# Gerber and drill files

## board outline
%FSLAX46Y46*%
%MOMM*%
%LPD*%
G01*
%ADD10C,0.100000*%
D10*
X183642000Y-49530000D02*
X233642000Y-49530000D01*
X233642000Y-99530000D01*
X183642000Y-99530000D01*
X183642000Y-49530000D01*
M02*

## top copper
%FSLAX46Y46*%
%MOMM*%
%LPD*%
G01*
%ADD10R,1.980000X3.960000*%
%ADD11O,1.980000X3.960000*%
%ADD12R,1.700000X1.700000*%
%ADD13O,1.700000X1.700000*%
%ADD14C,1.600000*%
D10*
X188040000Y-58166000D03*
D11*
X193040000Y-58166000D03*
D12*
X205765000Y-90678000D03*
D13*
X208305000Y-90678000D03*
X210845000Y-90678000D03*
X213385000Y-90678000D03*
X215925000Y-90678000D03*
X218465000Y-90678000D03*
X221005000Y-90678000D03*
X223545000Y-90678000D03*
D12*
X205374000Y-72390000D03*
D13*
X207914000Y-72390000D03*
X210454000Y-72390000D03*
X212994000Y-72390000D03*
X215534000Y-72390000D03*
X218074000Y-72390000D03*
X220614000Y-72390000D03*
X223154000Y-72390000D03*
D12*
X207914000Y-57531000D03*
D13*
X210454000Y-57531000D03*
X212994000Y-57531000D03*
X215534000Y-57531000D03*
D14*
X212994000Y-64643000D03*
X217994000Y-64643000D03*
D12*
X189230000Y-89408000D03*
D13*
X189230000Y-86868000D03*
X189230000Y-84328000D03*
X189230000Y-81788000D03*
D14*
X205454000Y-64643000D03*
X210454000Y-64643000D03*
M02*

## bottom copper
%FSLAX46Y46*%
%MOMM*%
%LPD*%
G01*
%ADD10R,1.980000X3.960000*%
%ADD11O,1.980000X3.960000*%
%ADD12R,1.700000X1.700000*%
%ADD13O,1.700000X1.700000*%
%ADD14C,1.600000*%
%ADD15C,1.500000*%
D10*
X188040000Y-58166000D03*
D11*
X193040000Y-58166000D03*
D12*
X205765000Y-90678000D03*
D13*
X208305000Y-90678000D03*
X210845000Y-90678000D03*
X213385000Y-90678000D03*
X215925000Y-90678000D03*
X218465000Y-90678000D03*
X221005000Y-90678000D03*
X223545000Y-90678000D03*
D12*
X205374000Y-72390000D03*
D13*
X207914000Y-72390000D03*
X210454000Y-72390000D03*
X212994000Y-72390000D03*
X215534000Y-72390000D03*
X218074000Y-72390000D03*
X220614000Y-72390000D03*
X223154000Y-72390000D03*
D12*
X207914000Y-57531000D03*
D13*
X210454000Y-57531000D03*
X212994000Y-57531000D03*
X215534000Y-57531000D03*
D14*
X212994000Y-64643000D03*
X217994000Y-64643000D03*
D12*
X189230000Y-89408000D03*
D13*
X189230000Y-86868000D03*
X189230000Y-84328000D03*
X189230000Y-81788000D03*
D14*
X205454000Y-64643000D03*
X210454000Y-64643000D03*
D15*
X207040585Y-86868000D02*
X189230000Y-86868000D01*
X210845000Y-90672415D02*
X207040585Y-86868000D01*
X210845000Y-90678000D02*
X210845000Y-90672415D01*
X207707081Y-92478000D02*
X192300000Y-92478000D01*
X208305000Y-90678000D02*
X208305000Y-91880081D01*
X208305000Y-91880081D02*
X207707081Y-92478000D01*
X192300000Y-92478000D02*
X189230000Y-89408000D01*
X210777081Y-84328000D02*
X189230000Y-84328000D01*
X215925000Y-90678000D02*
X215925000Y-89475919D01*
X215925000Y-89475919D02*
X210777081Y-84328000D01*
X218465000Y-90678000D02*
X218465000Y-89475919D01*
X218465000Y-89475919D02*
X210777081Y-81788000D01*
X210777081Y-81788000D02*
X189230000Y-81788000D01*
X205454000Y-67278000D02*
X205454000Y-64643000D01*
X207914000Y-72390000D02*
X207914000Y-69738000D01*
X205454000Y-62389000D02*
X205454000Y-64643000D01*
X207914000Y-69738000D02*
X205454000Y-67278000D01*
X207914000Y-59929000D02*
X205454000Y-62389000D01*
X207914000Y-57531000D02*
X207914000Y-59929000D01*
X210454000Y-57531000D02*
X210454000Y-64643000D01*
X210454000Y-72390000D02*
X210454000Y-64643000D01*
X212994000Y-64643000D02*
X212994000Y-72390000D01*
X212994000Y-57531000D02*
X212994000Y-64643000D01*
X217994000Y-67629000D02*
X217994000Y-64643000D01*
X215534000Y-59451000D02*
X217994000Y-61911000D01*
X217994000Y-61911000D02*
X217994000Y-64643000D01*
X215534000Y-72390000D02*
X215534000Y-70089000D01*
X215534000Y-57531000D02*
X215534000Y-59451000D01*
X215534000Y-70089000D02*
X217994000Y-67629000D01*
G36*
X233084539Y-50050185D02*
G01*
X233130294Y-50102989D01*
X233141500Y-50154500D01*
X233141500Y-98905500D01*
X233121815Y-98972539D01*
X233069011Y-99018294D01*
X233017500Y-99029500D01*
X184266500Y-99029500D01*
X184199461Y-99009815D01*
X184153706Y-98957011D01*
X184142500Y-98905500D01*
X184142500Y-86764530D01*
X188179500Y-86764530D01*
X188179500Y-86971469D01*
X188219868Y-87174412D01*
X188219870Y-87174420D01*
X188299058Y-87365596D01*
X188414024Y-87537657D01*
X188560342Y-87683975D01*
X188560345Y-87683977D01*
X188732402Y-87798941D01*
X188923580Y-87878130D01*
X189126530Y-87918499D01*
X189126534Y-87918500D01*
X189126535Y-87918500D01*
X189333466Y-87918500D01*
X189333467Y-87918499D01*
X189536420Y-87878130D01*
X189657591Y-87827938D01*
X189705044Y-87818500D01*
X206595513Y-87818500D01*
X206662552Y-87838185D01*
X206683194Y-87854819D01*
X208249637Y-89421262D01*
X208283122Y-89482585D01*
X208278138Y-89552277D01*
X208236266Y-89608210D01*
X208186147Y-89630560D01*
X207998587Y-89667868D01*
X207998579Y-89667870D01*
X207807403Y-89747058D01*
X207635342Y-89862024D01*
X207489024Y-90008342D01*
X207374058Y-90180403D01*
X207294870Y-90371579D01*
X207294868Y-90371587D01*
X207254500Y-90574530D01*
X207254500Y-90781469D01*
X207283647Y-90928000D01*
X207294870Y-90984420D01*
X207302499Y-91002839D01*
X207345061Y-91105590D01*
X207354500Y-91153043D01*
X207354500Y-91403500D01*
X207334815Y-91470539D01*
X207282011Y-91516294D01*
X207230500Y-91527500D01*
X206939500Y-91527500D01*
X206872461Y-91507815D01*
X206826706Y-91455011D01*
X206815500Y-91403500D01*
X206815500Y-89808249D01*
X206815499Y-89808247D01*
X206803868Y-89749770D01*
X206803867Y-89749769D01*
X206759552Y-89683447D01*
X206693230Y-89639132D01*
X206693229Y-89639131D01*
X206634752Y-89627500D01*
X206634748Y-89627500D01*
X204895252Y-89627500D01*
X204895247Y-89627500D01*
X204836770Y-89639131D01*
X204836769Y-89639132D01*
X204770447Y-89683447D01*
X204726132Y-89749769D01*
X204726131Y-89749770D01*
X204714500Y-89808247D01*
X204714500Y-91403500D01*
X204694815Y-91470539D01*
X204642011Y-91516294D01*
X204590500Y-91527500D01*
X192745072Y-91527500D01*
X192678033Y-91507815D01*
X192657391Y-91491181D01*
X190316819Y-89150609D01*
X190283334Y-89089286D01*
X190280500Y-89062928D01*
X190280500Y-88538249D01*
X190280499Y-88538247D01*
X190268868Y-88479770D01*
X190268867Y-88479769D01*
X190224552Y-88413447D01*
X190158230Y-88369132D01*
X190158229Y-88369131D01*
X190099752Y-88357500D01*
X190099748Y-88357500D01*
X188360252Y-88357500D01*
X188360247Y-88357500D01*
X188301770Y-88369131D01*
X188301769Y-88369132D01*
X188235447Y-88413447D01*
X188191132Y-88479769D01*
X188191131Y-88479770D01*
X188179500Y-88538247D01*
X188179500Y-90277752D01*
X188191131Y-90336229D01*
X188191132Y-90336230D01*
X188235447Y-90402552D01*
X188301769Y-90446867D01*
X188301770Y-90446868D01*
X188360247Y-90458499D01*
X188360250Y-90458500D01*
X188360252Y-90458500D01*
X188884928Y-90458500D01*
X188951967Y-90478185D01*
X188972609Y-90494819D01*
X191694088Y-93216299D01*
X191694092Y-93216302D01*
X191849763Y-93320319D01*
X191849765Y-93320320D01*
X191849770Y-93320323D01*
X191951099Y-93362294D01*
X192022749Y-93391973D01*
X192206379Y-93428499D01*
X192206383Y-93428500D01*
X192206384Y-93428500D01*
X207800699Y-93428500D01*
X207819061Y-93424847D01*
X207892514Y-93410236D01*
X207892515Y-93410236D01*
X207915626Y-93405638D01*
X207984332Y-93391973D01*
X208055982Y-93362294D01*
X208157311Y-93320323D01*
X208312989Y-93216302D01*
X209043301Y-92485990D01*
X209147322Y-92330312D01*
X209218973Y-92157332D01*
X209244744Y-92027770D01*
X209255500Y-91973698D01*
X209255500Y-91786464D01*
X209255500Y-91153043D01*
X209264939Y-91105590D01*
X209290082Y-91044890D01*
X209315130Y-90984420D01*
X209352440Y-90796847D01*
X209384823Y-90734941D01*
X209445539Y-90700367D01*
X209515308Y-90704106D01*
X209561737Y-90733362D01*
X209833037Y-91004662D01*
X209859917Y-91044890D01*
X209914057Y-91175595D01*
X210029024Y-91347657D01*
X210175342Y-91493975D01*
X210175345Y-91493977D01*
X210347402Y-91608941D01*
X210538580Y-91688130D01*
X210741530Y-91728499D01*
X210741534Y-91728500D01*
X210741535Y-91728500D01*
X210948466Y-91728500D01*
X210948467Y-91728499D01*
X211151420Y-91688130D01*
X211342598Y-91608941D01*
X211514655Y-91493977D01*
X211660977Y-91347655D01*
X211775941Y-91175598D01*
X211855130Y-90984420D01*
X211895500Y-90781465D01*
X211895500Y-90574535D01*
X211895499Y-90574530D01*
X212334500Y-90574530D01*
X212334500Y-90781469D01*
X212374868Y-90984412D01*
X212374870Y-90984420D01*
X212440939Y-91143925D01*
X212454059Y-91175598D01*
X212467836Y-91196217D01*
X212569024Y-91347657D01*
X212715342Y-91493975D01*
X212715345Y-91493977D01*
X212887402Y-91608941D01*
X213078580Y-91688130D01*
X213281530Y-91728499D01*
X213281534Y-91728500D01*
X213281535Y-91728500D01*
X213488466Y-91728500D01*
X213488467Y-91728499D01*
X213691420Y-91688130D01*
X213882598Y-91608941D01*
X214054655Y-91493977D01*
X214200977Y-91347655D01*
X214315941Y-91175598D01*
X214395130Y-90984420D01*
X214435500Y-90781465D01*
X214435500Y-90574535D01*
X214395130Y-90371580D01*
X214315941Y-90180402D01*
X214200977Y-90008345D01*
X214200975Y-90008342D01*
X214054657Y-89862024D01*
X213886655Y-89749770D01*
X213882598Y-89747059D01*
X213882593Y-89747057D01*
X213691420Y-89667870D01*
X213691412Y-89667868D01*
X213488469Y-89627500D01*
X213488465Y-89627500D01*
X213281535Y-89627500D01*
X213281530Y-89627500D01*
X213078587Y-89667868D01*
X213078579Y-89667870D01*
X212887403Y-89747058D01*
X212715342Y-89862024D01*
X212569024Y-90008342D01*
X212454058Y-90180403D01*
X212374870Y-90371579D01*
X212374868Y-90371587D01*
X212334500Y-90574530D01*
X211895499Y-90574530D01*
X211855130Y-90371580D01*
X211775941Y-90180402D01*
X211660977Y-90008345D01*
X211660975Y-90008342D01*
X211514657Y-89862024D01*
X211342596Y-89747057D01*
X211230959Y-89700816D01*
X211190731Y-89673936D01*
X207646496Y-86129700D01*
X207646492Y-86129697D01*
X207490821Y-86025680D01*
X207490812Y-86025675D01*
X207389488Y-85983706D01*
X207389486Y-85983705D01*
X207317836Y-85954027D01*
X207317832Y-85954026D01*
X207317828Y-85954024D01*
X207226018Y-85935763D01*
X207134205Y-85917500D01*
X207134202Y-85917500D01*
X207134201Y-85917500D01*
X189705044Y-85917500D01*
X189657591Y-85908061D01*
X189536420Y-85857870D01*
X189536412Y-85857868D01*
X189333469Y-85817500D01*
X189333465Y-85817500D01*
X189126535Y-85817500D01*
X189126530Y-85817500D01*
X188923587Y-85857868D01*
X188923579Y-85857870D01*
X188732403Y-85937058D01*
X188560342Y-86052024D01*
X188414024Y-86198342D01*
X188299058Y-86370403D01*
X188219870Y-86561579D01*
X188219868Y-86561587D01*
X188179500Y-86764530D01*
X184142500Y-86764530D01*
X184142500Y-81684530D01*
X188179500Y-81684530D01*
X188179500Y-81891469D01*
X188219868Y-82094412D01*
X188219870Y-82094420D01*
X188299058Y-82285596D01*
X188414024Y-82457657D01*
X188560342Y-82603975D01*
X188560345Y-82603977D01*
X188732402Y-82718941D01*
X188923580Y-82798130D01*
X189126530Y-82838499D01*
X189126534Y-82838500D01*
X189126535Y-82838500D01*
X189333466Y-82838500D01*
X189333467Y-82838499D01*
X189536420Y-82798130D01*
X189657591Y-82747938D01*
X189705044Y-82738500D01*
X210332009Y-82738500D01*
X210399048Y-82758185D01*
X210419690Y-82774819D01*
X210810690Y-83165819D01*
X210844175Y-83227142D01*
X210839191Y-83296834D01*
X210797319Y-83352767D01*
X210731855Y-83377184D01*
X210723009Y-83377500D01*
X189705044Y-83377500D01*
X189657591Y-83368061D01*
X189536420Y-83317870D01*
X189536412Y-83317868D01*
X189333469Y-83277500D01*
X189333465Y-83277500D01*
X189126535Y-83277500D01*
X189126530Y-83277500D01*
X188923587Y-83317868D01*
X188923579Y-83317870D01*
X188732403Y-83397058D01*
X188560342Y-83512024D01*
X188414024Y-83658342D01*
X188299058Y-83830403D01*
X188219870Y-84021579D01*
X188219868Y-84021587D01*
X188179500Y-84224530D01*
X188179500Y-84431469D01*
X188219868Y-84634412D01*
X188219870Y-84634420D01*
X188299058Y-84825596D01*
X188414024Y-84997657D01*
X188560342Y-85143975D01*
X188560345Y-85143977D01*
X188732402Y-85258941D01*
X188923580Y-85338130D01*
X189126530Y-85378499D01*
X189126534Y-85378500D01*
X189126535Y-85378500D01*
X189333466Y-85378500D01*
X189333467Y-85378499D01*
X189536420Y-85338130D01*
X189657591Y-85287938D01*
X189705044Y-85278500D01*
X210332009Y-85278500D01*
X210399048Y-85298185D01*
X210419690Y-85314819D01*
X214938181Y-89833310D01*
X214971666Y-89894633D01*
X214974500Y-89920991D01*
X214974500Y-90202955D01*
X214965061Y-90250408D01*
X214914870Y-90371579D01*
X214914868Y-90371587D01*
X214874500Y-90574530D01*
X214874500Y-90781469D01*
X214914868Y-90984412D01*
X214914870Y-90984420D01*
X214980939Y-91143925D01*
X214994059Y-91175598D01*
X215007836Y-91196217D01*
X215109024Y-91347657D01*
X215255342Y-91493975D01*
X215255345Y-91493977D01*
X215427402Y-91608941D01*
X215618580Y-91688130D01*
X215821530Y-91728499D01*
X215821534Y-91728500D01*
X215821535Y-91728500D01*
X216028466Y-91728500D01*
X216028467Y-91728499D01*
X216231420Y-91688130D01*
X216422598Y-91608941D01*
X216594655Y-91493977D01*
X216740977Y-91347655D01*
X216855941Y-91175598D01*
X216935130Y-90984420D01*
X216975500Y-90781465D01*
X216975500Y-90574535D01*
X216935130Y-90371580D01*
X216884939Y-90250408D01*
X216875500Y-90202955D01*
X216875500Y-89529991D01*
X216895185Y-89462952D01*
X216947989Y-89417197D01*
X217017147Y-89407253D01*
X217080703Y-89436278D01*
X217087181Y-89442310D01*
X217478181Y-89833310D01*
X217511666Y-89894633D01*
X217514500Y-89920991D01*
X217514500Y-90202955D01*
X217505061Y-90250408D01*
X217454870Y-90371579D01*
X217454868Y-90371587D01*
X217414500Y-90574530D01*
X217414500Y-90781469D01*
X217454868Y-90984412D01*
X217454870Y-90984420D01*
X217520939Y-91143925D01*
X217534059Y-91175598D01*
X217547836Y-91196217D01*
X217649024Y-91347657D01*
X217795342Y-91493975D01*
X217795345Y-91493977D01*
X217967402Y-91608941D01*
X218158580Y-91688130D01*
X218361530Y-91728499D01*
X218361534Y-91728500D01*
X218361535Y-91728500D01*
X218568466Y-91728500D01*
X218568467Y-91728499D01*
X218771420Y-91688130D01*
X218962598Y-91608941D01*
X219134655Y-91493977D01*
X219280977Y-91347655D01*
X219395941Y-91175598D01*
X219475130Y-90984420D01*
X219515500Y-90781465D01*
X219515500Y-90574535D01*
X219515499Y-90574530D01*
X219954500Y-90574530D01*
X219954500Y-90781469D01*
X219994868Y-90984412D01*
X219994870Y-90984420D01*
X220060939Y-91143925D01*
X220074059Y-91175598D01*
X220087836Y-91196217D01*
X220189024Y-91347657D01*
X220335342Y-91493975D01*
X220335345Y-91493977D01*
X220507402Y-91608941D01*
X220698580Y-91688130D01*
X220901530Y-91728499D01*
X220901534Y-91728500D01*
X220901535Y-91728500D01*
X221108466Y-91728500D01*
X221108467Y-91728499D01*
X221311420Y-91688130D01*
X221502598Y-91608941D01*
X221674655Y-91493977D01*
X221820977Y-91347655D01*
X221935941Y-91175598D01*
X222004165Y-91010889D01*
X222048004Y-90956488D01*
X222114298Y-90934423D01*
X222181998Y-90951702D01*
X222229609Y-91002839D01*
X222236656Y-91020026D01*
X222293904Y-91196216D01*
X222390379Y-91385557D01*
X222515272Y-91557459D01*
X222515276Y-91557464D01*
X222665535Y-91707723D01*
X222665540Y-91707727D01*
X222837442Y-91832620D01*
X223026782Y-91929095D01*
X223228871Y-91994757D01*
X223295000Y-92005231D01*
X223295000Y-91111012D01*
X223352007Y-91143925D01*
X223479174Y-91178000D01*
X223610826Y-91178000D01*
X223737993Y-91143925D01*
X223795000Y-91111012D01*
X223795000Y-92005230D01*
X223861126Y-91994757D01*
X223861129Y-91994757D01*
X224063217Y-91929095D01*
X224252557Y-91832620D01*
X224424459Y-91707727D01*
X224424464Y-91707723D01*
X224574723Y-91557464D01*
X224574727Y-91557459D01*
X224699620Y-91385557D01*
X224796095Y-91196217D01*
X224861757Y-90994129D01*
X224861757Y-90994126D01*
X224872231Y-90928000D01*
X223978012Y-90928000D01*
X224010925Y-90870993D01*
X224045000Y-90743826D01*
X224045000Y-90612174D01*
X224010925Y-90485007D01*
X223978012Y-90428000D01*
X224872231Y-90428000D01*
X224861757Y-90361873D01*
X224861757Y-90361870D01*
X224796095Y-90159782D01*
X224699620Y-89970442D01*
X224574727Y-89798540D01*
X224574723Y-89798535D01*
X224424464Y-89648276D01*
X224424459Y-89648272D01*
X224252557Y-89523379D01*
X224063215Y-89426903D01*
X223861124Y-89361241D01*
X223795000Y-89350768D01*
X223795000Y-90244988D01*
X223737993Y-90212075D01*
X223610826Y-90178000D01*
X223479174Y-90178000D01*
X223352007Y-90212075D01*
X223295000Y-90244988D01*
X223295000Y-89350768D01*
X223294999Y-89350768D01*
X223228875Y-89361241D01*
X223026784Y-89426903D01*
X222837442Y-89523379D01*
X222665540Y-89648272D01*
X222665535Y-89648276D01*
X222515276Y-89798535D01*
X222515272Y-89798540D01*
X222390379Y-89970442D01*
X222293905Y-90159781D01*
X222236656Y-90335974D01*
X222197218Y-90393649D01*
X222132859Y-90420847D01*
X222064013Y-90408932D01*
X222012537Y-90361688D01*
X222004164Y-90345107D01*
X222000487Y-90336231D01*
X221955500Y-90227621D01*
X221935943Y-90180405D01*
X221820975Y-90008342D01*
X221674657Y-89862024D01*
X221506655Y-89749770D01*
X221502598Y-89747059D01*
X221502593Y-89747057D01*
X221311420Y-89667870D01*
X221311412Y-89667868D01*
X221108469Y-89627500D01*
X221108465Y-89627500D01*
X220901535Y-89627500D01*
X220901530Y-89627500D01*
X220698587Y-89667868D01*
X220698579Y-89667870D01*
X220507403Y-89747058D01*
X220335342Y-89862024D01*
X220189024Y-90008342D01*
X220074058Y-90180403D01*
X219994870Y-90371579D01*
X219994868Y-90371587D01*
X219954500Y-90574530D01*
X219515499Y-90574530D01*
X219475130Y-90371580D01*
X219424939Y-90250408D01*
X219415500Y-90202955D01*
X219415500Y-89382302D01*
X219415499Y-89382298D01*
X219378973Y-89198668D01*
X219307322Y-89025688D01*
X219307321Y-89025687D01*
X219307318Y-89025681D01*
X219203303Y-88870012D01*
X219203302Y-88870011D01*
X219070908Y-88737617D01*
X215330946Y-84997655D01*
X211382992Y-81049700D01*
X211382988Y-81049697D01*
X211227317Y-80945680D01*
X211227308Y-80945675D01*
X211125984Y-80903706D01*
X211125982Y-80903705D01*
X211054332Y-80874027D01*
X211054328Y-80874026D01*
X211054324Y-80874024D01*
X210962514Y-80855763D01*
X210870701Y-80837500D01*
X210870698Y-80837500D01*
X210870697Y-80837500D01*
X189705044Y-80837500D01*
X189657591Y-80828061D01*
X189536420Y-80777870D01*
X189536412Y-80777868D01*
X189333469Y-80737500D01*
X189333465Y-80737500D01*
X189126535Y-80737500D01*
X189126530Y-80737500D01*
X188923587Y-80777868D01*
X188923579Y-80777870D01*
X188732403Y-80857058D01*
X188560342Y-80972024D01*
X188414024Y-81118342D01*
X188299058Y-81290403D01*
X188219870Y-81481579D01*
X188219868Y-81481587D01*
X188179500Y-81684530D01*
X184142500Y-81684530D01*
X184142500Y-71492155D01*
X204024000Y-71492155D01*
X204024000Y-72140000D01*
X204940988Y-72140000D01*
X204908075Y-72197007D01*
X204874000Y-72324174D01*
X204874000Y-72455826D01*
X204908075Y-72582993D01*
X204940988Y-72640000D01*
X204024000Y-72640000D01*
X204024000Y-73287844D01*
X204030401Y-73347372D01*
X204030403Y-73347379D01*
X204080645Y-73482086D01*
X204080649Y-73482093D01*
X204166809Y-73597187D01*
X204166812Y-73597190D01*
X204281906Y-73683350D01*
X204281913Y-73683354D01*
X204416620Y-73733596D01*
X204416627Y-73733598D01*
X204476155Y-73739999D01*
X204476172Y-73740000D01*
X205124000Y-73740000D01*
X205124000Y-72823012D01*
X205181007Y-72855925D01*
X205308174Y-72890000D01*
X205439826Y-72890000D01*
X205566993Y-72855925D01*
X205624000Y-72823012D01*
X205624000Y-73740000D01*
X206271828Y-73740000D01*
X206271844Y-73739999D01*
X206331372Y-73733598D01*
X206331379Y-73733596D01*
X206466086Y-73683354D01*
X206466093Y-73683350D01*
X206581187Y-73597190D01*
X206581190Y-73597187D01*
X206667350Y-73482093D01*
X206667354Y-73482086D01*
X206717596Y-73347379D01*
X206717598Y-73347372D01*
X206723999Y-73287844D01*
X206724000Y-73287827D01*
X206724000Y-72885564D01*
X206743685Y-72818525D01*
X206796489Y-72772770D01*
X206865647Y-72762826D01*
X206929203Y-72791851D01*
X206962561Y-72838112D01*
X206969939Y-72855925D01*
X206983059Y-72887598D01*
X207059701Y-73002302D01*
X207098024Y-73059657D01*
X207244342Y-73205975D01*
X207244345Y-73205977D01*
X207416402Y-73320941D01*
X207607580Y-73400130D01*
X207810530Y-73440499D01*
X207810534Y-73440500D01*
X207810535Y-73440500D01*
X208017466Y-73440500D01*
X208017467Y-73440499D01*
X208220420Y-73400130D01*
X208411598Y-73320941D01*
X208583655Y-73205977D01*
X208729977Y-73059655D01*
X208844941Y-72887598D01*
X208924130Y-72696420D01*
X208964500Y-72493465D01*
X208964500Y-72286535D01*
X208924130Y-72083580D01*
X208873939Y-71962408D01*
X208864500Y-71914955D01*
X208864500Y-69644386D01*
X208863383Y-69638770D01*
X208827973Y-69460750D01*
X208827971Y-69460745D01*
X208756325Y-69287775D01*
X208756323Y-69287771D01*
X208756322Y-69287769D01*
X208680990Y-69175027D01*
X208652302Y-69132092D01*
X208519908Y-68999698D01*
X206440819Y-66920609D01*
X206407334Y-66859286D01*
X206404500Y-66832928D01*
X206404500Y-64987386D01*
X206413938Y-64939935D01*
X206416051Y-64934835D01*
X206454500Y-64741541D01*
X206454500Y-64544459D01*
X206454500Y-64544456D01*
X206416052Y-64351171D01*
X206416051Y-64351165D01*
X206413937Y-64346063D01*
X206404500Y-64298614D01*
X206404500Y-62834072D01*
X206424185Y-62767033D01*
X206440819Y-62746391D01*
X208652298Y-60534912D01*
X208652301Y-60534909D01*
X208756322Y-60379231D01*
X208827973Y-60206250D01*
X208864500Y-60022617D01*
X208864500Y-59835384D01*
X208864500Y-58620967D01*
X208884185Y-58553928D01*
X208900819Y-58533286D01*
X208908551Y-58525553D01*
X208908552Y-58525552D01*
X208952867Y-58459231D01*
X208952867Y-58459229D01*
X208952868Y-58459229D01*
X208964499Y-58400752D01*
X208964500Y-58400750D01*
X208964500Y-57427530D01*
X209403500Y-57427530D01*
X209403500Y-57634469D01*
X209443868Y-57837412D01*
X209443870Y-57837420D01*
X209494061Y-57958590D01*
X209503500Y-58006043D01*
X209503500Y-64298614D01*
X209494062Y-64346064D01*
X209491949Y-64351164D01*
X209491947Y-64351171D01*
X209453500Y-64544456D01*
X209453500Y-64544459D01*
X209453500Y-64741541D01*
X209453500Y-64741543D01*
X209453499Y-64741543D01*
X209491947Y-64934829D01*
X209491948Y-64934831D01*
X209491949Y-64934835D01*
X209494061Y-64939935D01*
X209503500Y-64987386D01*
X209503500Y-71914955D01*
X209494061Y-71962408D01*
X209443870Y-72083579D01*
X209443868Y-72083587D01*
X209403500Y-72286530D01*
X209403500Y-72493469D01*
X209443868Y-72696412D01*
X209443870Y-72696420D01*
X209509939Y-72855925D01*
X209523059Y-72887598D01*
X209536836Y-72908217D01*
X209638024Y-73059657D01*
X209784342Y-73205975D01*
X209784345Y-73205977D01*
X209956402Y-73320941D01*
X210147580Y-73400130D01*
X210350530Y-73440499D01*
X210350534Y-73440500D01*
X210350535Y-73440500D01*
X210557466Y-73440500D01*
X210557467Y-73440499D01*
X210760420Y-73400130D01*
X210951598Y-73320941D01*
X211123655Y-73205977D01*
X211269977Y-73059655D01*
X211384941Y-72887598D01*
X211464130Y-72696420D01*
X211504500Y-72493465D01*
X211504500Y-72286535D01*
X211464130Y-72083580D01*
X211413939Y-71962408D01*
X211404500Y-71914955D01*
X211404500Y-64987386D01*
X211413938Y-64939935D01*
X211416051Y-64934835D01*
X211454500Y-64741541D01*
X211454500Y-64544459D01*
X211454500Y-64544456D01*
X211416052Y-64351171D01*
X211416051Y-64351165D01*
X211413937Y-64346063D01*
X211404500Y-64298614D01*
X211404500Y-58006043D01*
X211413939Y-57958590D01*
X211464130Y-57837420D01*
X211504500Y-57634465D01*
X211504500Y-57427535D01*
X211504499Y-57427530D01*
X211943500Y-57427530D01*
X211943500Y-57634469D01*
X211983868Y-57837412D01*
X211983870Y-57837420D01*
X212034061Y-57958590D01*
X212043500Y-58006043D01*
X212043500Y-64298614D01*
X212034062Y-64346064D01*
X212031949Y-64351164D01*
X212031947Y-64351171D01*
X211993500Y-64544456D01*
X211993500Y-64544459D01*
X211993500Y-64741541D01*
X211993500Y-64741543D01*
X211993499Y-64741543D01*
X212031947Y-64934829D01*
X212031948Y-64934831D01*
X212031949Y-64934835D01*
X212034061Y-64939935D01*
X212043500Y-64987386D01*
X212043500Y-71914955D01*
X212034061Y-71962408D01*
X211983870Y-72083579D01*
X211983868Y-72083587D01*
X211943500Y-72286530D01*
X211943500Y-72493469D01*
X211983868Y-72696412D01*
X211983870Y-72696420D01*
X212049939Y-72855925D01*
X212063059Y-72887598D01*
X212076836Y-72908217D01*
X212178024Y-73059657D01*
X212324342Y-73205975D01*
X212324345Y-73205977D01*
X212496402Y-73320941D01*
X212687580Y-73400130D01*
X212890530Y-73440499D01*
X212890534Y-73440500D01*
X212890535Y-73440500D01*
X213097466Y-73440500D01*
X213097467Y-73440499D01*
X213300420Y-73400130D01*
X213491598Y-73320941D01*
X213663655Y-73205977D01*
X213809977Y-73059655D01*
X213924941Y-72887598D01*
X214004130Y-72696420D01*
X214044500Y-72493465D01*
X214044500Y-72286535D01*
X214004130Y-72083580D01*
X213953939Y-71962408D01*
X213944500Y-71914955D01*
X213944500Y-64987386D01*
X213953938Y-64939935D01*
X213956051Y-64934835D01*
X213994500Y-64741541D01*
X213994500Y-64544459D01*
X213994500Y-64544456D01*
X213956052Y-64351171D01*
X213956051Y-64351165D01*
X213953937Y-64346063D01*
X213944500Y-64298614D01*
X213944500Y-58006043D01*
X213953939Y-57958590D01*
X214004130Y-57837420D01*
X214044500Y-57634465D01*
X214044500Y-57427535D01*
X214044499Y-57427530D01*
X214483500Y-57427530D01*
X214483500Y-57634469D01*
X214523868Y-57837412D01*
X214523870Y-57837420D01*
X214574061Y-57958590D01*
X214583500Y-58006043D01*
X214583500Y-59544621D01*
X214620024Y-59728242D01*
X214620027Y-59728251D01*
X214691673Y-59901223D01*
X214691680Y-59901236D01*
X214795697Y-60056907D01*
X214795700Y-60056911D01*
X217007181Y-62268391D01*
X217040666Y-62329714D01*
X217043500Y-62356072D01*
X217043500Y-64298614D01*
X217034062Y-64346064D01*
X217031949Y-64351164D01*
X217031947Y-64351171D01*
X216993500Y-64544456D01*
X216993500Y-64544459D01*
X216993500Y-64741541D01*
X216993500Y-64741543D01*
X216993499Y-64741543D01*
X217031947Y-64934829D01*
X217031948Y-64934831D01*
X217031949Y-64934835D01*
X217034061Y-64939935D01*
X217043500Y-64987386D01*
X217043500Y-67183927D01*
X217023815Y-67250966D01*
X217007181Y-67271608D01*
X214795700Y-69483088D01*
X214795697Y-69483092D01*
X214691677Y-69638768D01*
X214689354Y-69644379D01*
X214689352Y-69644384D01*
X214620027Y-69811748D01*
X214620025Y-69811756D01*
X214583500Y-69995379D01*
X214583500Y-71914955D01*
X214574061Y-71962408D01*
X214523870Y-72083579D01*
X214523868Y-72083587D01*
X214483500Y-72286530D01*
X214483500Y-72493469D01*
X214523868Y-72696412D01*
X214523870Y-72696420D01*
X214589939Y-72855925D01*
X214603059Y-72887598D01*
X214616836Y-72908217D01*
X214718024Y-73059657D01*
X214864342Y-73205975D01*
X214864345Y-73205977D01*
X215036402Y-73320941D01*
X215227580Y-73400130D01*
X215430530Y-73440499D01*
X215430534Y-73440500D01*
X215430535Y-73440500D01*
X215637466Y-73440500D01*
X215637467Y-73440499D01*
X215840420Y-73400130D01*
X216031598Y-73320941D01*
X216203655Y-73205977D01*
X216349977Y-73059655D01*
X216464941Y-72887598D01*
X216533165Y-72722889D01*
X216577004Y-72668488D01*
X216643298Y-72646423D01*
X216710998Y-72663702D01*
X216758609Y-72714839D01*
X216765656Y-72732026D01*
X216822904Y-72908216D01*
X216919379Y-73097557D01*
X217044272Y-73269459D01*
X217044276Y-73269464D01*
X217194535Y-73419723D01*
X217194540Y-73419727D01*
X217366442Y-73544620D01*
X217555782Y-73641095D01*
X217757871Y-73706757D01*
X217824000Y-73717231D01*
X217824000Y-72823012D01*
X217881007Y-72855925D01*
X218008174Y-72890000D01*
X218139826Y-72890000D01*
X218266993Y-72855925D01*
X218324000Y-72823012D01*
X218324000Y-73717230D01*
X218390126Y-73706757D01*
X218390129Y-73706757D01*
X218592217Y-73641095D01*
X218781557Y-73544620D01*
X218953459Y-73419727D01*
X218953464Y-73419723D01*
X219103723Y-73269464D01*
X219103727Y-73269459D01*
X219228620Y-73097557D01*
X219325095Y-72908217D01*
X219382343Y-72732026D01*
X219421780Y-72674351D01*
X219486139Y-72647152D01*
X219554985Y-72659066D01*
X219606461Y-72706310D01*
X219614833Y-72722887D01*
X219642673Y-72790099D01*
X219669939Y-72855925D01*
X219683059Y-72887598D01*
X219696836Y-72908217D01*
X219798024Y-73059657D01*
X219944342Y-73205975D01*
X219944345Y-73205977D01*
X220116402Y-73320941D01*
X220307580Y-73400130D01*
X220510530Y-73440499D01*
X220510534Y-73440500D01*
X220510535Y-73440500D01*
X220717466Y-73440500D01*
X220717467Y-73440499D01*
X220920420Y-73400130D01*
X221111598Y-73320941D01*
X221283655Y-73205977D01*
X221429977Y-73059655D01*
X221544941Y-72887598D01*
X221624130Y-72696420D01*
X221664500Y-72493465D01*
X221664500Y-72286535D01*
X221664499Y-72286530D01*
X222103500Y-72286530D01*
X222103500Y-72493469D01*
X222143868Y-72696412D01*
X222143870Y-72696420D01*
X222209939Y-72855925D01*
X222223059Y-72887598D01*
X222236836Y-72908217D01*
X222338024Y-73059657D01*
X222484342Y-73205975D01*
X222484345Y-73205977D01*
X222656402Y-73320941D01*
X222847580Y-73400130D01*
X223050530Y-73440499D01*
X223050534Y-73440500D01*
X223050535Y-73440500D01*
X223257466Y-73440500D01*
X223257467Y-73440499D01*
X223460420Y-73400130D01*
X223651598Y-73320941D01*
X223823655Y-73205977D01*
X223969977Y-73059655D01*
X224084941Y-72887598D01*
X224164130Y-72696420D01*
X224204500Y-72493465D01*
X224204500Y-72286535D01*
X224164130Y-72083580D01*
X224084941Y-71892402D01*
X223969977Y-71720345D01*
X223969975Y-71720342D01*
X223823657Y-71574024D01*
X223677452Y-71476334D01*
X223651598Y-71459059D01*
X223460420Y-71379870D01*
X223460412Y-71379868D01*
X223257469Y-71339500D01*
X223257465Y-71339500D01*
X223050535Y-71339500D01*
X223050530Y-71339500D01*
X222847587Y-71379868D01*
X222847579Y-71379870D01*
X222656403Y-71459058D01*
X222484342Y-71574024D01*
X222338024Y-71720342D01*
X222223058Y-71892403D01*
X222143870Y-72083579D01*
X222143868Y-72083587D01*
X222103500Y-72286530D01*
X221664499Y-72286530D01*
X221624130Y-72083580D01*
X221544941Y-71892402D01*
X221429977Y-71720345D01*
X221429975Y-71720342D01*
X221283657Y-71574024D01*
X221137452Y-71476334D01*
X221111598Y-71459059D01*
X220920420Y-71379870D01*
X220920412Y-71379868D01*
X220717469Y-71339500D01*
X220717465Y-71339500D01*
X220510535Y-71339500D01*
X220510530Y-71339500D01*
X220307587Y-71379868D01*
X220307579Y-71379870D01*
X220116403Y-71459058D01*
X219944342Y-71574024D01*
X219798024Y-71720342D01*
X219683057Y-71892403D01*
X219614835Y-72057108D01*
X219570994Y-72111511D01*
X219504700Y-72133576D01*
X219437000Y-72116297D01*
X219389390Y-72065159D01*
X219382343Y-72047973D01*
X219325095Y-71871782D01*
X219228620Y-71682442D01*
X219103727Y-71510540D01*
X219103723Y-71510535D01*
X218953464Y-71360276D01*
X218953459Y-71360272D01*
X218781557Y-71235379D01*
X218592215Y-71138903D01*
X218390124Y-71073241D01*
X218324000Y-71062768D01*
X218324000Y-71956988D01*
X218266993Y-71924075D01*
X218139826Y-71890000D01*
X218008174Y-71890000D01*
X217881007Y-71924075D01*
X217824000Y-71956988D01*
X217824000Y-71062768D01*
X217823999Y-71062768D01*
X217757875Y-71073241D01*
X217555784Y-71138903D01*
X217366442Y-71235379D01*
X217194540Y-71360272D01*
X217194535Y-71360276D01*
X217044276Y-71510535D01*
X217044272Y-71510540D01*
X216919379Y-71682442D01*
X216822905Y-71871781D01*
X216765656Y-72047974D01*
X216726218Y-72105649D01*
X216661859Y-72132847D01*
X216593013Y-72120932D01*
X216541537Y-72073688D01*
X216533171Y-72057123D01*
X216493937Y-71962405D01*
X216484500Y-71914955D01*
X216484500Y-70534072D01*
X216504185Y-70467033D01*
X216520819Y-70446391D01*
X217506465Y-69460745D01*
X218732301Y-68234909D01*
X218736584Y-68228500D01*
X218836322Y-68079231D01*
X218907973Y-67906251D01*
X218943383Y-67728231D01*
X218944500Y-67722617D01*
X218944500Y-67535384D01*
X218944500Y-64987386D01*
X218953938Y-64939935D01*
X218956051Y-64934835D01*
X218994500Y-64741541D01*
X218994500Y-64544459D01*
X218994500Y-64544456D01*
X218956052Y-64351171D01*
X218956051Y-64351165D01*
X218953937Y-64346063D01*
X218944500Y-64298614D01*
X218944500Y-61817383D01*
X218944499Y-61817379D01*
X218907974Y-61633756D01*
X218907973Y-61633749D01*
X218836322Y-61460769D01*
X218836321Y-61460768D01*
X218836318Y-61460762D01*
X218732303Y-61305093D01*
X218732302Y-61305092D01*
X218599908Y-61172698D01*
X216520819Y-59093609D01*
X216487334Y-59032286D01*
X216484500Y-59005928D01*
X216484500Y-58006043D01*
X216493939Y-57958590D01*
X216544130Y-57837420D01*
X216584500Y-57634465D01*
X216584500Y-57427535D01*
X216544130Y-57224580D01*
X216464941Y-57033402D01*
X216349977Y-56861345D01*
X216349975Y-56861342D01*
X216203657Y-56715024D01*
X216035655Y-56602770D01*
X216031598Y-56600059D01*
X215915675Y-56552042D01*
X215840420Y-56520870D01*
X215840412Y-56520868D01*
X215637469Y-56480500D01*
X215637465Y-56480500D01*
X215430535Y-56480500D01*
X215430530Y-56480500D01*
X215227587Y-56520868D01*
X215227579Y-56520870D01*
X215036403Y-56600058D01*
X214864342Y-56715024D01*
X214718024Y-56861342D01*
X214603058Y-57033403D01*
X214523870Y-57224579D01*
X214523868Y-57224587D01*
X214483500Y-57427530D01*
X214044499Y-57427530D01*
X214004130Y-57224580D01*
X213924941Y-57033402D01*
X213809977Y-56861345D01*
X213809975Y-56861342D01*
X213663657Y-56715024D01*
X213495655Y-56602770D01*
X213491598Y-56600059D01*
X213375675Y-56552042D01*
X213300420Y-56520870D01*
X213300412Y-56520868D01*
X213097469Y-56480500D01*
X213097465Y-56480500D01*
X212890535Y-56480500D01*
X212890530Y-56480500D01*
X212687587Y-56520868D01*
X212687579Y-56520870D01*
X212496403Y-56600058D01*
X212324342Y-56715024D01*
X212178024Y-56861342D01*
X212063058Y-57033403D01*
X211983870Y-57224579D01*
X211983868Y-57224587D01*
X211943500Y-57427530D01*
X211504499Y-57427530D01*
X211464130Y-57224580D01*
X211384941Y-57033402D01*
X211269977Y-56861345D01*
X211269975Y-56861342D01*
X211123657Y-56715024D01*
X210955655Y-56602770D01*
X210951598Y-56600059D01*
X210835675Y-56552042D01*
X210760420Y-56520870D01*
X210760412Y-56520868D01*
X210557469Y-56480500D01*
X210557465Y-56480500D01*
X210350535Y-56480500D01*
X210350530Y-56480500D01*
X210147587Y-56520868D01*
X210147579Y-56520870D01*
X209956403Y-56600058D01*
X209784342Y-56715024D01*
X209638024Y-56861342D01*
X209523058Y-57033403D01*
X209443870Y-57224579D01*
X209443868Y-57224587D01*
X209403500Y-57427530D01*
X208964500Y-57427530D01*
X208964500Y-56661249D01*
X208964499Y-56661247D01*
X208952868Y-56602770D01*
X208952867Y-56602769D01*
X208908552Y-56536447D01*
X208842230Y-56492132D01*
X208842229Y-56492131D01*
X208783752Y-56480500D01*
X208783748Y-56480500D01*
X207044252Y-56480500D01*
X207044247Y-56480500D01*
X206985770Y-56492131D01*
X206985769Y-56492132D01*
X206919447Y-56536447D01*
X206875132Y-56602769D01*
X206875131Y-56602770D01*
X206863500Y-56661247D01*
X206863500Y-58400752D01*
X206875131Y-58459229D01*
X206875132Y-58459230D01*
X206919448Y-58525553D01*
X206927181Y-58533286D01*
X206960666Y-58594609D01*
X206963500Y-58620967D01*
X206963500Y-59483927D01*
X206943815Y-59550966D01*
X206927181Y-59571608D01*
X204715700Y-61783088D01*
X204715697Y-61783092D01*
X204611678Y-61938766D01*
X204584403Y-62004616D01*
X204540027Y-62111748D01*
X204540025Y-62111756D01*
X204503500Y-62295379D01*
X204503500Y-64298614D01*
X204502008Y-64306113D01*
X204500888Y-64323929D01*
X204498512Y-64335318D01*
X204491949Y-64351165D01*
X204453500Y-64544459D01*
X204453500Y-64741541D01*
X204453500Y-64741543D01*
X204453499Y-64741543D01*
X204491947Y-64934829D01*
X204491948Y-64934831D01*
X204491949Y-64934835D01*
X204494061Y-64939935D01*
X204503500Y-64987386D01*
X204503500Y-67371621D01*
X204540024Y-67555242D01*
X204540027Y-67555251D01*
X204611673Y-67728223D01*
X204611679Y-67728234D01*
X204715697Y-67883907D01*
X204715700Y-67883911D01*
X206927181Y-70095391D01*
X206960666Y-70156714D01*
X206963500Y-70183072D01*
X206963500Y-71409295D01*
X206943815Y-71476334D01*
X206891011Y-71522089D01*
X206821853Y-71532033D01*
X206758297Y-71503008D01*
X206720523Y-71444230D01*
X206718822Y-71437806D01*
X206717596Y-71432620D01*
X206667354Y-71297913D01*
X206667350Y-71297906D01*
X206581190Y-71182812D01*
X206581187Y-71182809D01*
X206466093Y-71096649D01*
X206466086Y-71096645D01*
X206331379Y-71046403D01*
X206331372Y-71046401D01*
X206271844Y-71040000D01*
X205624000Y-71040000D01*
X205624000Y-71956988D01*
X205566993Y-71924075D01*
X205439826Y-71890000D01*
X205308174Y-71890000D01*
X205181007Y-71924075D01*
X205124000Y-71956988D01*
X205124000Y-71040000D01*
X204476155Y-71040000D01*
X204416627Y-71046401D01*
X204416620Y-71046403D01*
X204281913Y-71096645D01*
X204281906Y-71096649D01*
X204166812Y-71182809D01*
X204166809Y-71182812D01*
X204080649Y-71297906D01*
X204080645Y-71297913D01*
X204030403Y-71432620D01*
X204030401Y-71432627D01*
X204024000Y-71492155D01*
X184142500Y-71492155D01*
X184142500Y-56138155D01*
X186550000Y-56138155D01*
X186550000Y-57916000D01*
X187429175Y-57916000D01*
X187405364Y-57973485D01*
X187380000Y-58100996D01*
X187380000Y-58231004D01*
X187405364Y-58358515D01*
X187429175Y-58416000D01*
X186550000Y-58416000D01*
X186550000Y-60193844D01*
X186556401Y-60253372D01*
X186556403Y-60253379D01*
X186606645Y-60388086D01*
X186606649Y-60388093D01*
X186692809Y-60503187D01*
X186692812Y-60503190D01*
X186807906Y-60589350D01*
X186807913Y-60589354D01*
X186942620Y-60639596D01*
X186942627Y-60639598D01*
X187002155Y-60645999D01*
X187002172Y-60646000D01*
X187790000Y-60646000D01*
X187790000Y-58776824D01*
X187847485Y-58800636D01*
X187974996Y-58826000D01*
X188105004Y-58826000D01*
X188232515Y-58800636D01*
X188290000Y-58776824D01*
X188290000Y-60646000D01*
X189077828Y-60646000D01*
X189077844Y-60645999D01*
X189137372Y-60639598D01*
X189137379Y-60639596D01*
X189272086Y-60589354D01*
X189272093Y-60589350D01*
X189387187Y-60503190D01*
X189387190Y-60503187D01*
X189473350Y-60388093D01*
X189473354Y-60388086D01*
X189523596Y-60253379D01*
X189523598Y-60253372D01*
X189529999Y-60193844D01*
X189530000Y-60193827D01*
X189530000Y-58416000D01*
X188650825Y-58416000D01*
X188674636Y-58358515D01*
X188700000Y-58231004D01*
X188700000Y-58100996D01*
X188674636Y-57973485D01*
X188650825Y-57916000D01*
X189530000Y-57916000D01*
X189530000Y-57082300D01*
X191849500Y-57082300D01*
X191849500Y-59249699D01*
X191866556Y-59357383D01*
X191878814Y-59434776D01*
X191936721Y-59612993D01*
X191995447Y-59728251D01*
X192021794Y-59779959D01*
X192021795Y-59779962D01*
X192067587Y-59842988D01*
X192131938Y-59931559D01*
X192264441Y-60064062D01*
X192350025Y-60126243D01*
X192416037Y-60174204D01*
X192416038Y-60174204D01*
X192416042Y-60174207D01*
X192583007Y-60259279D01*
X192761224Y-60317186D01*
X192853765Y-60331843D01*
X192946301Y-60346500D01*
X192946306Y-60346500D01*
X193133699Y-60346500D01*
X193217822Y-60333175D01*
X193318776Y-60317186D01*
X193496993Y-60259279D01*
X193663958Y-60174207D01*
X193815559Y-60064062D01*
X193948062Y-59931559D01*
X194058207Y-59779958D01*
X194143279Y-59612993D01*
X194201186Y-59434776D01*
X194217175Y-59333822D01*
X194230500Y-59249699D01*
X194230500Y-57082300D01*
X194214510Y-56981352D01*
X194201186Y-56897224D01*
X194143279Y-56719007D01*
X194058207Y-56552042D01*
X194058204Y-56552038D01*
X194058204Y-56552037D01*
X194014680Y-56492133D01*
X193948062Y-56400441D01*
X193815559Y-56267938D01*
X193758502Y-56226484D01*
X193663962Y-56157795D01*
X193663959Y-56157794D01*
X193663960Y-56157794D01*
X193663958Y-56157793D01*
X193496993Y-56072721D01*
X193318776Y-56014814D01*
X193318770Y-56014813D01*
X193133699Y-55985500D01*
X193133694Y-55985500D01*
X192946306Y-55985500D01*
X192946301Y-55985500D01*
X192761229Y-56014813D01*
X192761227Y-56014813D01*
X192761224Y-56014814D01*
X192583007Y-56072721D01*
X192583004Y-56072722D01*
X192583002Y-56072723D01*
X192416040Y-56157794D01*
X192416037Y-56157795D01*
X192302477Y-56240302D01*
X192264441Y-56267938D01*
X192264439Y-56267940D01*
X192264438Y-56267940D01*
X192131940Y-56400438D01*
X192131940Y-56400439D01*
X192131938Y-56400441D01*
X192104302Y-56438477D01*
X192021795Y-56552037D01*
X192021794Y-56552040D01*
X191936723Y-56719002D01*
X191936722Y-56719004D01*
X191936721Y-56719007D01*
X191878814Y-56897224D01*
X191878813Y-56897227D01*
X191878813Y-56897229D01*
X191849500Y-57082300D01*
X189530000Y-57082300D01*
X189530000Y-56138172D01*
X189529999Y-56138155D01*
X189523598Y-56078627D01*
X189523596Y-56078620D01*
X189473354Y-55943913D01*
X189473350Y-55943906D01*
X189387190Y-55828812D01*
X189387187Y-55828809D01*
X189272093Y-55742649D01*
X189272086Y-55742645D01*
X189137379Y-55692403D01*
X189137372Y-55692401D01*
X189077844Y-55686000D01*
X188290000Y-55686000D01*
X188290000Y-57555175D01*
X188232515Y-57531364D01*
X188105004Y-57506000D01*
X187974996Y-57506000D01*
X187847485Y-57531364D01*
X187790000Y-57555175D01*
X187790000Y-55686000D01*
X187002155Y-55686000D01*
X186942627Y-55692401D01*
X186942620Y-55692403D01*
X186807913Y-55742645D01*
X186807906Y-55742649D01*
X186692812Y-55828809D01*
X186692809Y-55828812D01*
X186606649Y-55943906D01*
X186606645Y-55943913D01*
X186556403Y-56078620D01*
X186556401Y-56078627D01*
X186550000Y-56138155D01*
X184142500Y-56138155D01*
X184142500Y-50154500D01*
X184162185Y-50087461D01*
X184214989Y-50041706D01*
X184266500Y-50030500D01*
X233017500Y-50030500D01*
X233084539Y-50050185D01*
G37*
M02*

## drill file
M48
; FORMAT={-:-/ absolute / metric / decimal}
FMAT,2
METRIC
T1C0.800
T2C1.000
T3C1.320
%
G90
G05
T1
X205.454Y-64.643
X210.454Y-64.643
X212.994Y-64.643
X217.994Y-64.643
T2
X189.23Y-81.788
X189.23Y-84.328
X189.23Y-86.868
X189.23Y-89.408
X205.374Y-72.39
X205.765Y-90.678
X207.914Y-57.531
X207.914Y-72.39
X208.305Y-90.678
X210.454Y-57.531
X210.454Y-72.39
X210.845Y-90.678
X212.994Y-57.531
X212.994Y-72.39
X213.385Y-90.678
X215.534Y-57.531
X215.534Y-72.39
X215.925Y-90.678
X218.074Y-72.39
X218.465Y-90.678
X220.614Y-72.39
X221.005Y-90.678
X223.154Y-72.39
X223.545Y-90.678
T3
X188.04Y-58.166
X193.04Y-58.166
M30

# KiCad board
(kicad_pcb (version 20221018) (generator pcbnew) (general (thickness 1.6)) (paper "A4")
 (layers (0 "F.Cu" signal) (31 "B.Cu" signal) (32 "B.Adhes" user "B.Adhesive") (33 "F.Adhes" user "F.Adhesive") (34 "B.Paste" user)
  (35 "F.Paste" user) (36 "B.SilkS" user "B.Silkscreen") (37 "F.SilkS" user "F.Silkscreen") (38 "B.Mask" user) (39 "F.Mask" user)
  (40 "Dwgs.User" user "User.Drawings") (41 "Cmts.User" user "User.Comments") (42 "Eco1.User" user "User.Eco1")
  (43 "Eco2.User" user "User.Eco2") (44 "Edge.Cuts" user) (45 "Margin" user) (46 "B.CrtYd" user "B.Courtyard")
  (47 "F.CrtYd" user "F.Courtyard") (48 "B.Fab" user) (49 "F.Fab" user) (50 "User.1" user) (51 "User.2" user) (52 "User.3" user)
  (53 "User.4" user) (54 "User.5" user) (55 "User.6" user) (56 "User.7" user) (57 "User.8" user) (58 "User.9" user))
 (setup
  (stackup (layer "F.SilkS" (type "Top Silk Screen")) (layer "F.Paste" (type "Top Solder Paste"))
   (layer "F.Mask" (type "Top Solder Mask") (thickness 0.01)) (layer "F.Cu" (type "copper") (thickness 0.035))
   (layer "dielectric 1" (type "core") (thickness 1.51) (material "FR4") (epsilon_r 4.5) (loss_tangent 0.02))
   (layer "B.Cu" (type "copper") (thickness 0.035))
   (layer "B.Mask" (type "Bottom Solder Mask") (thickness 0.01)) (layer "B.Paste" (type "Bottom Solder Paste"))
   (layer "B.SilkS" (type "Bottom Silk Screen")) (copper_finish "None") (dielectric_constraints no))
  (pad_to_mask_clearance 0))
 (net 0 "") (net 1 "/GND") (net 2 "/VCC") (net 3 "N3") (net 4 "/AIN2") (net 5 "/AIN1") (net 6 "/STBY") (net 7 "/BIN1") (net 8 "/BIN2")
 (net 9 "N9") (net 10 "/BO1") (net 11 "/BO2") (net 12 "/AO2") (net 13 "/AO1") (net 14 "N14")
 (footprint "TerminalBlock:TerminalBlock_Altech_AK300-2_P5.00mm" (layer "F.Cu") (at 188.04 58.166)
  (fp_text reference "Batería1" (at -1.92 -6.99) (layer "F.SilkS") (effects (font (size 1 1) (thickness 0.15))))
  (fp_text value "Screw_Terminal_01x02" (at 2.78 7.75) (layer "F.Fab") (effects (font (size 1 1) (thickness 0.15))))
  (pad "1" thru_hole rect (at 0 0) (size 1.98 3.96) (drill 1.32) (layers "*.Cu" "*.Mask") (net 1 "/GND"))
  (pad "2" thru_hole oval (at 5 0) (size 1.98 3.96) (drill 1.32) (layers "*.Cu" "*.Mask") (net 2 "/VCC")))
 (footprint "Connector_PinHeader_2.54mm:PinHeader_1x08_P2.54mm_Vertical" (layer "F.Cu") (at 205.765 90.678 90)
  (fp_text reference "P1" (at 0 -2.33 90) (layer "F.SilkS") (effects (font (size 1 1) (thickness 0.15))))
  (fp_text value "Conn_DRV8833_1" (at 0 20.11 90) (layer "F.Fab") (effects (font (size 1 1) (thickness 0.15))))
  (pad "1" thru_hole rect (at 0 0 90) (size 1.7 1.7) (drill 1) (layers "*.Cu" "*.Mask") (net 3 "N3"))
  (pad "2" thru_hole oval (at 0 2.54 90) (size 1.7 1.7) (drill 1) (layers "*.Cu" "*.Mask") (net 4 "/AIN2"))
  (pad "3" thru_hole oval (at 0 5.08 90) (size 1.7 1.7) (drill 1) (layers "*.Cu" "*.Mask") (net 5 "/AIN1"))
  (pad "4" thru_hole oval (at 0 7.62 90) (size 1.7 1.7) (drill 1) (layers "*.Cu" "*.Mask") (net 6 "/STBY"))
  (pad "5" thru_hole oval (at 0 10.16 90) (size 1.7 1.7) (drill 1) (layers "*.Cu" "*.Mask") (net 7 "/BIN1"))
  (pad "6" thru_hole oval (at 0 12.7 90) (size 1.7 1.7) (drill 1) (layers "*.Cu" "*.Mask") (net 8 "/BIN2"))
  (pad "7" thru_hole oval (at 0 15.24 90) (size 1.7 1.7) (drill 1) (layers "*.Cu" "*.Mask") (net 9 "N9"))
  (pad "8" thru_hole oval (at 0 17.78 90) (size 1.7 1.7) (drill 1) (layers "*.Cu" "*.Mask") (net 1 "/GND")))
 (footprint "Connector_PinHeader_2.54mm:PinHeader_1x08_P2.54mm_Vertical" (layer "F.Cu") (at 205.374 72.39 90)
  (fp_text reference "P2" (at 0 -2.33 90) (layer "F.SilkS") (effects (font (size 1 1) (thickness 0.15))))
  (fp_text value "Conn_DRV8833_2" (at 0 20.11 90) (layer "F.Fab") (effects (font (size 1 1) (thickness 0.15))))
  (pad "1" thru_hole rect (at 0 0 90) (size 1.7 1.7) (drill 1) (layers "*.Cu" "*.Mask") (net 1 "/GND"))
  (pad "2" thru_hole oval (at 0 2.54 90) (size 1.7 1.7) (drill 1) (layers "*.Cu" "*.Mask") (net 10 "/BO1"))
  (pad "3" thru_hole oval (at 0 5.08 90) (size 1.7 1.7) (drill 1) (layers "*.Cu" "*.Mask") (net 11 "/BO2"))
  (pad "4" thru_hole oval (at 0 7.62 90) (size 1.7 1.7) (drill 1) (layers "*.Cu" "*.Mask") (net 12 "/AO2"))
  (pad "5" thru_hole oval (at 0 10.16 90) (size 1.7 1.7) (drill 1) (layers "*.Cu" "*.Mask") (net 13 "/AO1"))
  (pad "6" thru_hole oval (at 0 12.7 90) (size 1.7 1.7) (drill 1) (layers "*.Cu" "*.Mask") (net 1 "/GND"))
  (pad "7" thru_hole oval (at 0 15.24 90) (size 1.7 1.7) (drill 1) (layers "*.Cu" "*.Mask") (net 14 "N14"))
  (pad "8" thru_hole oval (at 0 17.78 90) (size 1.7 1.7) (drill 1) (layers "*.Cu" "*.Mask") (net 2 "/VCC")))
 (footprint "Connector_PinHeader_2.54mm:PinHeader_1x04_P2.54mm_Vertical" (layer "F.Cu") (at 207.914 57.531 90)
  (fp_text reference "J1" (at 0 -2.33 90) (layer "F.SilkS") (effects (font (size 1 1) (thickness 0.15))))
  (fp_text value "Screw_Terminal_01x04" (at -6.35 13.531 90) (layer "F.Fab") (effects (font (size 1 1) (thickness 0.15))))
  (pad "1" thru_hole rect (at 0 0 90) (size 1.7 1.7) (drill 1) (layers "*.Cu" "*.Mask") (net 10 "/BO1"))
  (pad "2" thru_hole oval (at 0 2.54 90) (size 1.7 1.7) (drill 1) (layers "*.Cu" "*.Mask") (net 11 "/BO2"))
  (pad "3" thru_hole oval (at 0 5.08 90) (size 1.7 1.7) (drill 1) (layers "*.Cu" "*.Mask") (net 12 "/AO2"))
  (pad "4" thru_hole oval (at 0 7.62 90) (size 1.7 1.7) (drill 1) (layers "*.Cu" "*.Mask") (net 13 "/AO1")))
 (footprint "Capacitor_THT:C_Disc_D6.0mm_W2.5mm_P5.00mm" (layer "F.Cu") (at 212.994 64.643)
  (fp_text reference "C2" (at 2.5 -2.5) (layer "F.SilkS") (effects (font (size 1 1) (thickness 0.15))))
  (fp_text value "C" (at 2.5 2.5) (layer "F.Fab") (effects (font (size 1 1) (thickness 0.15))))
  (pad "1" thru_hole circle (at 0 0) (size 1.6 1.6) (drill 0.8) (layers "*.Cu" "*.Mask") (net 12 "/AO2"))
  (pad "2" thru_hole circle (at 5 0) (size 1.6 1.6) (drill 0.8) (layers "*.Cu" "*.Mask") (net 13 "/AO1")))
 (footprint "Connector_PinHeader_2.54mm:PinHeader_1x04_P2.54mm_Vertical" (layer "F.Cu") (at 189.23 89.408 180)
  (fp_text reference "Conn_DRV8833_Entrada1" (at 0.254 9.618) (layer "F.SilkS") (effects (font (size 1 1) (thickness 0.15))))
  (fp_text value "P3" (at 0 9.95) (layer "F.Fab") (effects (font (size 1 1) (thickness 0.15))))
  (pad "1" thru_hole rect (at 0 0 180) (size 1.7 1.7) (drill 1) (layers "*.Cu" "*.Mask") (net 4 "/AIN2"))
  (pad "2" thru_hole oval (at 0 2.54 180) (size 1.7 1.7) (drill 1) (layers "*.Cu" "*.Mask") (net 5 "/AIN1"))
  (pad "3" thru_hole oval (at 0 5.08 180) (size 1.7 1.7) (drill 1) (layers "*.Cu" "*.Mask") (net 7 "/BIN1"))
  (pad "4" thru_hole oval (at 0 7.62 180) (size 1.7 1.7) (drill 1) (layers "*.Cu" "*.Mask") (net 8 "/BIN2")))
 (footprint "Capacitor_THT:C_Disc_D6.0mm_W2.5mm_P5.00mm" (layer "F.Cu") (at 205.454 64.643)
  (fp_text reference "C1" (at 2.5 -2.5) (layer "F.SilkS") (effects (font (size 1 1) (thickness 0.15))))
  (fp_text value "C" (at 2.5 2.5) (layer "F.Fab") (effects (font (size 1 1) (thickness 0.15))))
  (pad "1" thru_hole circle (at 0 0) (size 1.6 1.6) (drill 0.8) (layers "*.Cu" "*.Mask") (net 10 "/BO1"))
  (pad "2" thru_hole circle (at 5 0) (size 1.6 1.6) (drill 0.8) (layers "*.Cu" "*.Mask") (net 11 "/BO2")))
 (gr_rect (start 183.642 49.53) (end 233.642 99.53) (stroke (width 0.1) (type default)) (fill none) (layer "Edge.Cuts"))
 (segment (start 207.040585 86.868) (end 189.23 86.868) (width 1.5) (layer "B.Cu") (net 5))
 (segment (start 210.845 90.672415) (end 207.040585 86.868) (width 1.5) (layer "B.Cu") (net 5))
 (segment (start 210.845 90.678) (end 210.845 90.672415) (width 1.5) (layer "B.Cu") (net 5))
 (segment (start 207.707081 92.478) (end 192.3 92.478) (width 1.5) (layer "B.Cu") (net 4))
 (segment (start 208.305 90.678) (end 208.305 91.880081) (width 1.5) (layer "B.Cu") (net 4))
 (segment (start 208.305 91.880081) (end 207.707081 92.478) (width 1.5) (layer "B.Cu") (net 4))
 (segment (start 192.3 92.478) (end 189.23 89.408) (width 1.5) (layer "B.Cu") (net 4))
 (segment (start 210.777081 84.328) (end 189.23 84.328) (width 1.5) (layer "B.Cu") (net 7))
 (segment (start 215.925 90.678) (end 215.925 89.475919) (width 1.5) (layer "B.Cu") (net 7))
 (segment (start 215.925 89.475919) (end 210.777081 84.328) (width 1.5) (layer "B.Cu") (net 7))
 (segment (start 218.465 90.678) (end 218.465 89.475919) (width 1.5) (layer "B.Cu") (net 8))
 (segment (start 218.465 89.475919) (end 210.777081 81.788) (width 1.5) (layer "B.Cu") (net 8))
 (segment (start 210.777081 81.788) (end 189.23 81.788) (width 1.5) (layer "B.Cu") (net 8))
 (segment (start 205.454 67.278) (end 205.454 64.643) (width 1.5) (layer "B.Cu") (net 10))
 (segment (start 207.914 72.39) (end 207.914 69.738) (width 1.5) (layer "B.Cu") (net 10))
 (segment (start 205.454 62.389) (end 205.454 64.643) (width 1.5) (layer "B.Cu") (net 10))
 (segment (start 207.914 69.738) (end 205.454 67.278) (width 1.5) (layer "B.Cu") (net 10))
 (segment (start 207.914 59.929) (end 205.454 62.389) (width 1.5) (layer "B.Cu") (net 10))
 (segment (start 207.914 57.531) (end 207.914 59.929) (width 1.5) (layer "B.Cu") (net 10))
 (segment (start 210.454 57.531) (end 210.454 64.643) (width 1.5) (layer "B.Cu") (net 11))
 (segment (start 210.454 72.39) (end 210.454 64.643) (width 1.5) (layer "B.Cu") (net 11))
 (segment (start 212.994 64.643) (end 212.994 72.39) (width 1.5) (layer "B.Cu") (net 12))
 (segment (start 212.994 57.531) (end 212.994 64.643) (width 1.5) (layer "B.Cu") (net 12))
 (segment (start 217.994 67.629) (end 217.994 64.643) (width 1.5) (layer "B.Cu") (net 13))
 (segment (start 215.534 59.451) (end 217.994 61.911) (width 1.5) (layer "B.Cu") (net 13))
 (segment (start 217.994 61.911) (end 217.994 64.643) (width 1.5) (layer "B.Cu") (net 13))
 (segment (start 215.534 72.39) (end 215.534 70.089) (width 1.5) (layer "B.Cu") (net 13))
 (segment (start 215.534 57.531) (end 215.534 59.451) (width 1.5) (layer "B.Cu") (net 13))
 (segment (start 215.534 70.089) (end 217.994 67.629) (width 1.5) (layer "B.Cu") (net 13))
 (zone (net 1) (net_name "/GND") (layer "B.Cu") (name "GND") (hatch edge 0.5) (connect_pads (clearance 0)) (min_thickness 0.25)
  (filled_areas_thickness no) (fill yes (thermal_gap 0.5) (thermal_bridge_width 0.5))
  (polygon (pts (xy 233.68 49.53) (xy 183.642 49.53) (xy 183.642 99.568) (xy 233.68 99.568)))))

